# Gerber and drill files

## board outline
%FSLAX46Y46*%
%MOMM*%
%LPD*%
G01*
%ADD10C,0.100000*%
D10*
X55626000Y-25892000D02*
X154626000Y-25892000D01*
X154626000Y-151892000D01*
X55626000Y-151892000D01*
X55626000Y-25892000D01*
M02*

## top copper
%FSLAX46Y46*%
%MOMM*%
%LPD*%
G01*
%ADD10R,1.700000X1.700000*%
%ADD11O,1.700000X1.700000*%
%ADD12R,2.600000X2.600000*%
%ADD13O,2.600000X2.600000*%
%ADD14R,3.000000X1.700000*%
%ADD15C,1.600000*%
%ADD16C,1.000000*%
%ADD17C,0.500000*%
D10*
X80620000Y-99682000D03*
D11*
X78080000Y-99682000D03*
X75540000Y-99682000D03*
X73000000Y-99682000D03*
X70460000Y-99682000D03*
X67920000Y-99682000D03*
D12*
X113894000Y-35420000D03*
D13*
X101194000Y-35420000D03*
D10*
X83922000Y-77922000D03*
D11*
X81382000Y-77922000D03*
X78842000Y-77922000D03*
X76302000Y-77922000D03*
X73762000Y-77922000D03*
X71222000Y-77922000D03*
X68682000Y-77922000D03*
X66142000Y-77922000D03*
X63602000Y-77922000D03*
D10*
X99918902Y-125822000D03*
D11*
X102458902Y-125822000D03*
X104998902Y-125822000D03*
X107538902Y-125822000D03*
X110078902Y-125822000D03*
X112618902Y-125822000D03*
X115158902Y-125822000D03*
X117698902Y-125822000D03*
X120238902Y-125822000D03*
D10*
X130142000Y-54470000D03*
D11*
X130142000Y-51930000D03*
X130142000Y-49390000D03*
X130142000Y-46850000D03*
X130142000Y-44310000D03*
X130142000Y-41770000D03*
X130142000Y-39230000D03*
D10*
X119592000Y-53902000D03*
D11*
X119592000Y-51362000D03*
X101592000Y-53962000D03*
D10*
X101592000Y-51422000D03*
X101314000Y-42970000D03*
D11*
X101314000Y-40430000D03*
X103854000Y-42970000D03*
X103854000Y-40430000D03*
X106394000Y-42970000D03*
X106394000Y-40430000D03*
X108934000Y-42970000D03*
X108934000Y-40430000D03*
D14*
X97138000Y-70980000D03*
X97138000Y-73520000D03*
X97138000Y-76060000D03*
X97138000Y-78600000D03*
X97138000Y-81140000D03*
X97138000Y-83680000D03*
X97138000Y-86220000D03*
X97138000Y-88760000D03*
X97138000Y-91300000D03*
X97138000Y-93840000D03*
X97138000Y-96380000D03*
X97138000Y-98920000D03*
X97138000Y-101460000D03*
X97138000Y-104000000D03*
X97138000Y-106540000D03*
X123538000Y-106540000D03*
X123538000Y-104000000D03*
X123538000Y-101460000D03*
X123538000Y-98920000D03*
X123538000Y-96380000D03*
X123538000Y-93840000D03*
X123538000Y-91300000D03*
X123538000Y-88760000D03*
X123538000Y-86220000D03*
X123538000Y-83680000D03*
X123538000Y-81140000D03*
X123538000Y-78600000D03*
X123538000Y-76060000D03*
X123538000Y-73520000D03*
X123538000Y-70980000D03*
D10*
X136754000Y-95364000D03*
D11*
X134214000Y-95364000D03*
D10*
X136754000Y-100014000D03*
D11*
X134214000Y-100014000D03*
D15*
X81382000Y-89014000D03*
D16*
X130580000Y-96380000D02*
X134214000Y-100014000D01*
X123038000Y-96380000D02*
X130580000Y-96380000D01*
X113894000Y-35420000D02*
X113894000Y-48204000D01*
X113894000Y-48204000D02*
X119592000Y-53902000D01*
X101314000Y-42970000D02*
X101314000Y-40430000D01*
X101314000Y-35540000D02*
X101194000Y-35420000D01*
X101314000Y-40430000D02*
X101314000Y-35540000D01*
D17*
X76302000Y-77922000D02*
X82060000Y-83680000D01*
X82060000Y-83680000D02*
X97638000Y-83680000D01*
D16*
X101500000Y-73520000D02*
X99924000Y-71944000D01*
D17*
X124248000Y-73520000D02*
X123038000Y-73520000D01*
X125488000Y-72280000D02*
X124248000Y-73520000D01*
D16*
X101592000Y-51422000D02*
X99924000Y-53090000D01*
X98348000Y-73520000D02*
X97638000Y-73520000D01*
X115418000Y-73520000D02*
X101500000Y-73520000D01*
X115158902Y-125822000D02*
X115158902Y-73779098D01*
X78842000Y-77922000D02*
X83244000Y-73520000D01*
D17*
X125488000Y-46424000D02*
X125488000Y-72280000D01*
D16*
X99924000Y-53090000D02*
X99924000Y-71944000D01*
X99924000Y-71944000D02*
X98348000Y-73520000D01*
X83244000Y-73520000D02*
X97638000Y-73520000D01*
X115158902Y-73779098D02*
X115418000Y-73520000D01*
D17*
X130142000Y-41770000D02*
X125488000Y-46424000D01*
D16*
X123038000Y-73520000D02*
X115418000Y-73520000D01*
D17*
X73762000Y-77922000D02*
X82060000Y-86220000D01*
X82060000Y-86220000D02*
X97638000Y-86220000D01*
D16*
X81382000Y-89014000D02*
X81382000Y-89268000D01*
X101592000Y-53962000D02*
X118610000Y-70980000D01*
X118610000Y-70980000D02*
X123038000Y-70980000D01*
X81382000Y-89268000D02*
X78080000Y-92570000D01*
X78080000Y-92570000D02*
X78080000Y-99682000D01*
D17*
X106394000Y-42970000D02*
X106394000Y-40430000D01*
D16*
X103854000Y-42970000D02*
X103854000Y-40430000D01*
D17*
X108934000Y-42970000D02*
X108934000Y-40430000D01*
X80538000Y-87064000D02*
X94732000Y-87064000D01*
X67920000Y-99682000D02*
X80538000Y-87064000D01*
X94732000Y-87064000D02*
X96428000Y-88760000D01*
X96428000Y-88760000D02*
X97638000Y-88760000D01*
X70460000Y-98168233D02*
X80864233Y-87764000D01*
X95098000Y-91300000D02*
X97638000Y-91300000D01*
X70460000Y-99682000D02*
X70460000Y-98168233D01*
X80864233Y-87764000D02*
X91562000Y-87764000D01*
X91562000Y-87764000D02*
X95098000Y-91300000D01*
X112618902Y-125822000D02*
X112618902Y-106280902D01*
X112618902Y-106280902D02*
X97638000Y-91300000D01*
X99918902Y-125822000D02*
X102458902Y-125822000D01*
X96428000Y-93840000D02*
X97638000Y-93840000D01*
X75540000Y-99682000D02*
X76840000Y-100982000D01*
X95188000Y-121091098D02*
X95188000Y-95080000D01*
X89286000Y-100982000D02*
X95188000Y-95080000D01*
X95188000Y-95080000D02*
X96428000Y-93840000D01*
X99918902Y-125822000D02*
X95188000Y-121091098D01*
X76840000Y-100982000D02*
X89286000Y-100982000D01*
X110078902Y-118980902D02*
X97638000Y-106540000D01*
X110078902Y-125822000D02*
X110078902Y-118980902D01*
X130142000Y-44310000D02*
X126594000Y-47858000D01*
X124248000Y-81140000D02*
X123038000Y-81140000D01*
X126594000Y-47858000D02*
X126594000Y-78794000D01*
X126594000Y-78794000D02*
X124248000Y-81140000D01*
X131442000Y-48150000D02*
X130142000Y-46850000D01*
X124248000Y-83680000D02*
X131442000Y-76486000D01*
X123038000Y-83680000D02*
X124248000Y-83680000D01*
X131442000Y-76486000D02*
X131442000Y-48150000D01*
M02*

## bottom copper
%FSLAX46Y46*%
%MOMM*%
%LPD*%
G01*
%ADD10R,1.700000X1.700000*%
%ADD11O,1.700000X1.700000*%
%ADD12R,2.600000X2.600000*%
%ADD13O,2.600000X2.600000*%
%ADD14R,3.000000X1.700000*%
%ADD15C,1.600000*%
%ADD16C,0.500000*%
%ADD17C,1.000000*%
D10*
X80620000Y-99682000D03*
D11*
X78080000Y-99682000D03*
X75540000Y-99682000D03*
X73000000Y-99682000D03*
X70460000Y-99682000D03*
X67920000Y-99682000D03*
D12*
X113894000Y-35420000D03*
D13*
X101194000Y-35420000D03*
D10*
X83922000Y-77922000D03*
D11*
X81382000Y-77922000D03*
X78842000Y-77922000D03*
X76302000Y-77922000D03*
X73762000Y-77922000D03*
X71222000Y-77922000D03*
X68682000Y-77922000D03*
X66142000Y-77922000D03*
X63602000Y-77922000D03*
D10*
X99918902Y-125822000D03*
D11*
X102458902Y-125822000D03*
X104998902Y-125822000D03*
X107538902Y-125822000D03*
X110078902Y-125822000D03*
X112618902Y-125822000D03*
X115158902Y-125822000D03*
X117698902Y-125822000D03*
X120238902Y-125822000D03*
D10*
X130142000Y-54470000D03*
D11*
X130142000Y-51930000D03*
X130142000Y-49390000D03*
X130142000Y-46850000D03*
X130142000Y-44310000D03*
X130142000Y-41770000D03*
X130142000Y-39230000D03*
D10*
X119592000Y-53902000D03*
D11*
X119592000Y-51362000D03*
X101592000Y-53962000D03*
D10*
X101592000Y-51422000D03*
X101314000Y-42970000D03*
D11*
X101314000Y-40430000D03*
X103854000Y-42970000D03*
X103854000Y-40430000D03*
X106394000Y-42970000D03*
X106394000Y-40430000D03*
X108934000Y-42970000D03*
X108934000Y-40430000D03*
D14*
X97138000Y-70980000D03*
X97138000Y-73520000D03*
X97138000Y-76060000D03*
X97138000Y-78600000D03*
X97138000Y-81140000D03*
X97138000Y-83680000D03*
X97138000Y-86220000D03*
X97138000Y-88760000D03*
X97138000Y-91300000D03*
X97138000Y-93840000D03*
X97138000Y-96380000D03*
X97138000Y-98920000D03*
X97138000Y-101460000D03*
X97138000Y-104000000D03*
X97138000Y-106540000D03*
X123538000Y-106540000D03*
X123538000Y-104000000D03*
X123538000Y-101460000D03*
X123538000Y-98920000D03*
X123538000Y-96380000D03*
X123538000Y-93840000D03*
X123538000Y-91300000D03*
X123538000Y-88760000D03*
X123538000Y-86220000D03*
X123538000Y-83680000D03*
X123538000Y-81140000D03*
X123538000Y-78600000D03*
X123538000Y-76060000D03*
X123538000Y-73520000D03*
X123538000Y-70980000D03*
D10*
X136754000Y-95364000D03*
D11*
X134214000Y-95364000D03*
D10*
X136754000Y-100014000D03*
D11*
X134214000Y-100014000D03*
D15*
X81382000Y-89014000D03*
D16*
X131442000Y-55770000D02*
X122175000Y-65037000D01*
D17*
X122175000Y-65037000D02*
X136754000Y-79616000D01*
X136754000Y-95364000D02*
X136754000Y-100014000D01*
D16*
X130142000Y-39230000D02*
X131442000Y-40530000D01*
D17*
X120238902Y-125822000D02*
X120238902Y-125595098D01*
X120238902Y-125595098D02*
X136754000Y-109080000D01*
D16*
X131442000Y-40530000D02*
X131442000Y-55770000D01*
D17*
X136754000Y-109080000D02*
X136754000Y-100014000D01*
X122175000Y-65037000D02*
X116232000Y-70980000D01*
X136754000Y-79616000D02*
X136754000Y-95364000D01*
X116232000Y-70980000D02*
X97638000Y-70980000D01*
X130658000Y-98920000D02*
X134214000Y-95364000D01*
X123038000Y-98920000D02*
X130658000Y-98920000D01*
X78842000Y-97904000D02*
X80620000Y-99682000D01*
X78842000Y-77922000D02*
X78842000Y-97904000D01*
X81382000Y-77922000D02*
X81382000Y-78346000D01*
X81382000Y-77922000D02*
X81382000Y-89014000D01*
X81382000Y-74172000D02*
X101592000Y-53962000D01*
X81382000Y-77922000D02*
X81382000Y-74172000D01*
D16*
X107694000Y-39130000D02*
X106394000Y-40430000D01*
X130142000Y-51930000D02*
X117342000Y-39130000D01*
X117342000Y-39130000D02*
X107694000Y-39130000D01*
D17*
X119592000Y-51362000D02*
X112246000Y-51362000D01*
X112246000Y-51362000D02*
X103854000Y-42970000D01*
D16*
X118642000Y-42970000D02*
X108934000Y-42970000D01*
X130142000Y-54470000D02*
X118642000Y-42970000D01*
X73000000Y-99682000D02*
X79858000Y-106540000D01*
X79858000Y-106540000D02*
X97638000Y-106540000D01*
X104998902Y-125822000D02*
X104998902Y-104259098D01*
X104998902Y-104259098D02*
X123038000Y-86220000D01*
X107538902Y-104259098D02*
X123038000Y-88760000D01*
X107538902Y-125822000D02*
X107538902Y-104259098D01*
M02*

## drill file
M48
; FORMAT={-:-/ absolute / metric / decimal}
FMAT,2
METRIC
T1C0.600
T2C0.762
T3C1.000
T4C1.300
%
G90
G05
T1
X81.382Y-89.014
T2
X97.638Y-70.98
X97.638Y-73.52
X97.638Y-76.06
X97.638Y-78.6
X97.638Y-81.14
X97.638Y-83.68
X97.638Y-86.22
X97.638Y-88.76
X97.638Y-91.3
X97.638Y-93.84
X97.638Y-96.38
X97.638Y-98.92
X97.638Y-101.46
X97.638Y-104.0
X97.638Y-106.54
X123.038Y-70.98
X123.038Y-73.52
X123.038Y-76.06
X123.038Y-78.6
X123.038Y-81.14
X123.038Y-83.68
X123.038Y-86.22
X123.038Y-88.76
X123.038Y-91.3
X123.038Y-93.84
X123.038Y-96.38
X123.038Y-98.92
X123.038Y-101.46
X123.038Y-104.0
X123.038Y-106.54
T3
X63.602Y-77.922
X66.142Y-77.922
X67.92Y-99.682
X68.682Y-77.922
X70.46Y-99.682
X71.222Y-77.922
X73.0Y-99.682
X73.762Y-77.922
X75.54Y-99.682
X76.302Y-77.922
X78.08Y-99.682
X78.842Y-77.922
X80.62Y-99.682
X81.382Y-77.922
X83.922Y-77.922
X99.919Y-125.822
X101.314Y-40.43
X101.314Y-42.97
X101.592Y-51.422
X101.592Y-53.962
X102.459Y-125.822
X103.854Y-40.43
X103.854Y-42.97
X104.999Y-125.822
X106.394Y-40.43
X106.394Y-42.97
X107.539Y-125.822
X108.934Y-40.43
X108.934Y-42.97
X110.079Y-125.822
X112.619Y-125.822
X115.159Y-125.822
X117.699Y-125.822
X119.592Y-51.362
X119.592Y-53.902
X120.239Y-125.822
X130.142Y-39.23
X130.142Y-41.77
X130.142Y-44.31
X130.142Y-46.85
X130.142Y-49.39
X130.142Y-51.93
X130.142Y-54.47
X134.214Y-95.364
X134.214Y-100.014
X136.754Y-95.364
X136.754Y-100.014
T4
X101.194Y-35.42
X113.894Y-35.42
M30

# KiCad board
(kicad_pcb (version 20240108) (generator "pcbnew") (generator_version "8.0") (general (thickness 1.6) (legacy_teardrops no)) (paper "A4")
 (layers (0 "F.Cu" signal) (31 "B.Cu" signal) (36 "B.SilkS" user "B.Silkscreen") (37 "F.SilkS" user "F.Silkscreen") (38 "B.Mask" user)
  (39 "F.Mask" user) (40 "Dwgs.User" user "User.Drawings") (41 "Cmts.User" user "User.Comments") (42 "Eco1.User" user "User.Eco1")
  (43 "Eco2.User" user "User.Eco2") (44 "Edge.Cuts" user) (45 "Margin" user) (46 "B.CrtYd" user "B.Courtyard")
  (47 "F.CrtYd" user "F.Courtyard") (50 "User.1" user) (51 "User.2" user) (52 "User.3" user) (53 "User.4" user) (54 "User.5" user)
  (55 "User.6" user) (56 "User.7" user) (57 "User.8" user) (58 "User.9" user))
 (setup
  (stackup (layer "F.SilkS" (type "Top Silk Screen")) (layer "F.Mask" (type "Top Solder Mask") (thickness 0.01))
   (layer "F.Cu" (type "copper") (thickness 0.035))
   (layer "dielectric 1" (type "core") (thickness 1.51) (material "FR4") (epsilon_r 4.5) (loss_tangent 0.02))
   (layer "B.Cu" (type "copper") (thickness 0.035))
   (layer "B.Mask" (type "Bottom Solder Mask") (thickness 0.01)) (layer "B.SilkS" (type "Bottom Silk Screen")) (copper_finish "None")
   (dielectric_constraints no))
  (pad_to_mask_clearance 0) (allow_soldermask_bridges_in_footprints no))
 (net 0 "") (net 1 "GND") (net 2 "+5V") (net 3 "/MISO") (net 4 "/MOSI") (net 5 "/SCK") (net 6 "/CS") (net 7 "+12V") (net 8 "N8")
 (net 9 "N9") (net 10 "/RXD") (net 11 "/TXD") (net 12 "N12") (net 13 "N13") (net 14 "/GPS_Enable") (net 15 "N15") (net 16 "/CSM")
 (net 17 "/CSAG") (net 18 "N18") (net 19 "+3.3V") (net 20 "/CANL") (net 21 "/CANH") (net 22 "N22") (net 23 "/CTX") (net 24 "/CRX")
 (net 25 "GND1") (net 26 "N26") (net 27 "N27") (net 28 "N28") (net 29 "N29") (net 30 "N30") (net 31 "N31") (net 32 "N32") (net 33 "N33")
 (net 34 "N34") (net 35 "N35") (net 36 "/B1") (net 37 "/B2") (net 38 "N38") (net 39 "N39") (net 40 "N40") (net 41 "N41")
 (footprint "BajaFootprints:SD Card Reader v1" (layer "F.Cu") (at 74.27 117.462 90)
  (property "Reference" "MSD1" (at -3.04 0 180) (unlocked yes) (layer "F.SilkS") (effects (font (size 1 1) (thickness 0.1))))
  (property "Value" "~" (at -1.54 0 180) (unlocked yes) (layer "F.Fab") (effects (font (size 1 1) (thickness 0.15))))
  (pad "1" thru_hole rect (at 17.78 6.35 270) (size 1.7 1.7) (drill 1) (layers "*.Cu" "*.Mask") (remove_unused_layers no) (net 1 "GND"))
  (pad "2" thru_hole oval (at 17.78 3.81 270) (size 1.7 1.7) (drill 1) (layers "*.Cu" "*.Mask") (remove_unused_layers no) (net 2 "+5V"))
  (pad "3" thru_hole oval (at 17.78 1.27 270) (size 1.7 1.7) (drill 1) (layers "*.Cu" "*.Mask") (remove_unused_layers no) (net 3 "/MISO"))
  (pad "4" thru_hole oval (at 17.78 -1.27 270) (size 1.7 1.7) (drill 1) (layers "*.Cu" "*.Mask") (remove_unused_layers no) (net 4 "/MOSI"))
  (pad "5" thru_hole oval (at 17.78 -3.81 270) (size 1.7 1.7) (drill 1) (layers "*.Cu" "*.Mask") (remove_unused_layers no) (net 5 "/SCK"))
  (pad "6" thru_hole oval (at 17.78 -6.35 270) (size 1.7 1.7) (drill 1) (layers "*.Cu" "*.Mask") (remove_unused_layers no) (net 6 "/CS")))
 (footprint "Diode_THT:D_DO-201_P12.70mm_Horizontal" (layer "F.Cu") (at 113.894 35.42 180)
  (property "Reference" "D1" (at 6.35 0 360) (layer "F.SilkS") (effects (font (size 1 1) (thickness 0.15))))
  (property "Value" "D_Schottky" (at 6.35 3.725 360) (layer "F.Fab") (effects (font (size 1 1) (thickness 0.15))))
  (pad "1" thru_hole rect (at 0 0 180) (size 2.6 2.6) (drill 1.3) (layers "*.Cu" "*.Mask") (remove_unused_layers no) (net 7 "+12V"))
  (pad "2" thru_hole oval (at 12.7 0 180) (size 2.6 2.6) (drill 1.3) (layers "*.Cu" "*.Mask") (remove_unused_layers no) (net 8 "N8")))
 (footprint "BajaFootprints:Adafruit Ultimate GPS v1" (layer "F.Cu") (at 73.762 62.852 -90)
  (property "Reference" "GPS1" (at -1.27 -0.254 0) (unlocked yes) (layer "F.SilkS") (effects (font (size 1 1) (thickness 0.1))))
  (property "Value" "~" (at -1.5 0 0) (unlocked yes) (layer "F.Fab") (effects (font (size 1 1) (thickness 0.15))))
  (pad "1" thru_hole rect (at 15.07 -10.16 270) (size 1.7 1.7) (drill 1) (layers "*.Cu" "*.Mask") (remove_unused_layers no) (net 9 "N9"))
  (pad "2" thru_hole oval (at 15.07 -7.62 270) (size 1.7 1.7) (drill 1) (layers "*.Cu" "*.Mask") (remove_unused_layers no) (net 2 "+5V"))
  (pad "3" thru_hole oval (at 15.07 -5.08 270) (size 1.7 1.7) (drill 1) (layers "*.Cu" "*.Mask") (remove_unused_layers no) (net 1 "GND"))
  (pad "4" thru_hole oval (at 15.07 -2.54 270) (size 1.7 1.7) (drill 1) (layers "*.Cu" "*.Mask") (remove_unused_layers no) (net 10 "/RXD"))
  (pad "5" thru_hole oval (at 15.07 0 270) (size 1.7 1.7) (drill 1) (layers "*.Cu" "*.Mask") (remove_unused_layers no) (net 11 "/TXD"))
  (pad "6" thru_hole oval (at 15.07 2.54 270) (size 1.7 1.7) (drill 1) (layers "*.Cu" "*.Mask") (remove_unused_layers no) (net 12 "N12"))
  (pad "7" thru_hole oval (at 15.07 5.08 270) (size 1.7 1.7) (drill 1) (layers "*.Cu" "*.Mask") (remove_unused_layers no) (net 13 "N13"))
  (pad "8" thru_hole oval (at 15.07 7.62 270) (size 1.7 1.7) (drill 1) (layers "*.Cu" "*.Mask") (remove_unused_layers no)
   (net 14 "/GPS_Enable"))
  (pad "9" thru_hole oval (at 15.07 10.16 270) (size 1.7 1.7) (drill 1) (layers "*.Cu" "*.Mask") (remove_unused_layers no) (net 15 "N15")))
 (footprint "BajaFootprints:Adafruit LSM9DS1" (layer "F.Cu") (at 110.084 133.972 90)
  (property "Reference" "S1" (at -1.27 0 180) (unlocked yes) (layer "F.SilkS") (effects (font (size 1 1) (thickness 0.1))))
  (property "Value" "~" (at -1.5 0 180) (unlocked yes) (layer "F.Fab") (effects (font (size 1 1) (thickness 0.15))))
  (pad "1" thru_hole rect (at 8.15 -10.165098 90) (size 1.7 1.7) (drill 1) (layers "*.Cu" "*.Mask") (remove_unused_layers no)
   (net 3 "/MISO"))
  (pad "2" thru_hole oval (at 8.15 -7.625098 90) (size 1.7 1.7) (drill 1) (layers "*.Cu" "*.Mask") (remove_unused_layers no) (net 3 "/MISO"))
  (pad "3" thru_hole oval (at 8.15 -5.085098 90) (size 1.7 1.7) (drill 1) (layers "*.Cu" "*.Mask") (remove_unused_layers no) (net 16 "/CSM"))
  (pad "4" thru_hole oval (at 8.15 -2.545098 90) (size 1.7 1.7) (drill 1) (layers "*.Cu" "*.Mask") (remove_unused_layers no)
   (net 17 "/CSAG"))
  (pad "5" thru_hole oval (at 8.15 -0.005098 90) (size 1.7 1.7) (drill 1) (layers "*.Cu" "*.Mask") (remove_unused_layers no) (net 4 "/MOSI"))
  (pad "6" thru_hole oval (at 8.15 2.534902 90) (size 1.7 1.7) (drill 1) (layers "*.Cu" "*.Mask") (remove_unused_layers no) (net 5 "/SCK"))
  (pad "7" thru_hole oval (at 8.15 5.074902 90) (size 1.7 1.7) (drill 1) (layers "*.Cu" "*.Mask") (remove_unused_layers no) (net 1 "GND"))
  (pad "8" thru_hole oval (at 8.15 7.614902 90) (size 1.7 1.7) (drill 1) (layers "*.Cu" "*.Mask") (remove_unused_layers no) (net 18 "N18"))
  (pad "9" thru_hole oval (at 8.15 10.154902 90) (size 1.7 1.7) (drill 1) (layers "*.Cu" "*.Mask") (remove_unused_layers no)
   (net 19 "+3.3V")))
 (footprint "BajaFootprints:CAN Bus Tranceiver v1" (layer "F.Cu") (at 138.532 46.85 180)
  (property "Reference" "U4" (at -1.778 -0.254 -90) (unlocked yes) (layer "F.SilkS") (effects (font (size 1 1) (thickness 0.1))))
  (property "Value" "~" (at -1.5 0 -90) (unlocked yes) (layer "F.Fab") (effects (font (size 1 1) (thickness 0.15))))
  (pad "1" thru_hole rect (at 8.39 -7.62 180) (size 1.7 1.7) (drill 1) (layers "*.Cu" "*.Mask") (remove_unused_layers no) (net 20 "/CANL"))
  (pad "2" thru_hole oval (at 8.39 -5.08 180) (size 1.7 1.7) (drill 1) (layers "*.Cu" "*.Mask") (remove_unused_layers no) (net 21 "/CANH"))
  (pad "3" thru_hole oval (at 8.39 -2.54 180) (size 1.7 1.7) (drill 1) (layers "*.Cu" "*.Mask") (remove_unused_layers no) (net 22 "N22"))
  (pad "4" thru_hole oval (at 8.39 0 180) (size 1.7 1.7) (drill 1) (layers "*.Cu" "*.Mask") (remove_unused_layers no) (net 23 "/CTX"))
  (pad "5" thru_hole oval (at 8.39 2.54 180) (size 1.7 1.7) (drill 1) (layers "*.Cu" "*.Mask") (remove_unused_layers no) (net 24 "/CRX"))
  (pad "6" thru_hole oval (at 8.39 5.08 180) (size 1.7 1.7) (drill 1) (layers "*.Cu" "*.Mask") (remove_unused_layers no) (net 1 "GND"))
  (pad "7" thru_hole oval (at 8.39 7.62 180) (size 1.7 1.7) (drill 1) (layers "*.Cu" "*.Mask") (remove_unused_layers no) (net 19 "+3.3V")))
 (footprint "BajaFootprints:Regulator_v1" (layer "F.Cu") (at 110.592 52.692 180)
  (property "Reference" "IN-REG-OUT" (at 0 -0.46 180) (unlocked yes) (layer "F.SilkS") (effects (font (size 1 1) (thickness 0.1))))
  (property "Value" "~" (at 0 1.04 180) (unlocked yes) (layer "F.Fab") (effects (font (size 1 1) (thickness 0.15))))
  (pad "1" thru_hole rect (at -9 -1.21 180) (size 1.7 1.7) (drill 1) (layers "*.Cu" "*.Mask") (remove_unused_layers no) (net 7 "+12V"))
  (pad "2" thru_hole oval (at -9 1.33 180) (size 1.7 1.7) (drill 1) (layers "*.Cu" "*.Mask") (remove_unused_layers no) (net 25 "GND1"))
  (pad "3" thru_hole oval (at 9 -1.27) (size 1.7 1.7) (drill 1) (layers "*.Cu" "*.Mask") (remove_unused_layers no) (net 2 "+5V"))
  (pad "4" thru_hole rect (at 9 1.27) (size 1.7 1.7) (drill 1) (layers "*.Cu" "*.Mask") (remove_unused_layers no) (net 1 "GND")))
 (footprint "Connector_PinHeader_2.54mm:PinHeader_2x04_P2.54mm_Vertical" (layer "F.Cu") (at 101.314 42.97 90)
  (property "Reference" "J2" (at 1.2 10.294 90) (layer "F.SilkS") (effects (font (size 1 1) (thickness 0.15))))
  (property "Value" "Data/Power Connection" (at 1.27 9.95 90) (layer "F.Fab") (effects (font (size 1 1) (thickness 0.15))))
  (pad "1" thru_hole rect (at 0 0 90) (size 1.7 1.7) (drill 1) (layers "*.Cu" "*.Mask") (remove_unused_layers no) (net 8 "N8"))
  (pad "2" thru_hole oval (at 2.54 0 90) (size 1.7 1.7) (drill 1) (layers "*.Cu" "*.Mask") (remove_unused_layers no) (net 8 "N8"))
  (pad "3" thru_hole oval (at 0 2.54 90) (size 1.7 1.7) (drill 1) (layers "*.Cu" "*.Mask") (remove_unused_layers no) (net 25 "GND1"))
  (pad "4" thru_hole oval (at 2.54 2.54 90) (size 1.7 1.7) (drill 1) (layers "*.Cu" "*.Mask") (remove_unused_layers no) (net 25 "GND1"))
  (pad "5" thru_hole oval (at 0 5.08 90) (size 1.7 1.7) (drill 1) (layers "*.Cu" "*.Mask") (remove_unused_layers no) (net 21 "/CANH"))
  (pad "6" thru_hole oval (at 2.54 5.08 90) (size 1.7 1.7) (drill 1) (layers "*.Cu" "*.Mask") (remove_unused_layers no) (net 21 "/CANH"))
  (pad "7" thru_hole oval (at 0 7.62 90) (size 1.7 1.7) (drill 1) (layers "*.Cu" "*.Mask") (remove_unused_layers no) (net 20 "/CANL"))
  (pad "8" thru_hole oval (at 2.54 7.62 90) (size 1.7 1.7) (drill 1) (layers "*.Cu" "*.Mask") (remove_unused_layers no) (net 20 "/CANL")))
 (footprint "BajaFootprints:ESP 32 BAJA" (layer "F.Cu") (at 110.338 70.98)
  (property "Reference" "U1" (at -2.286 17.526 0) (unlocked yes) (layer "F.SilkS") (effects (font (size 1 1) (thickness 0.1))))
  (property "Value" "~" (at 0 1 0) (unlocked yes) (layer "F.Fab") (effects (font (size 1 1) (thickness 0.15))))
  (pad "1" thru_hole rect (at -12.7 0) (size 3 1.7) (drill 0.762 (offset -0.5 0)) (layers "*.Cu" "*.Mask") (remove_unused_layers no)
   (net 19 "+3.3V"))
  (pad "2" thru_hole rect (at -12.7 2.54) (size 3 1.7) (drill 0.762 (offset -0.5 0)) (layers "*.Cu" "*.Mask") (remove_unused_layers no)
   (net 1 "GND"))
  (pad "3" thru_hole rect (at -12.7 5.08) (size 3 1.7) (drill 0.762 (offset -0.5 0)) (layers "*.Cu" "*.Mask") (remove_unused_layers no)
   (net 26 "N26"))
  (pad "4" thru_hole rect (at -12.7 7.62) (size 3 1.7) (drill 0.762 (offset -0.5 0)) (layers "*.Cu" "*.Mask") (remove_unused_layers no)
   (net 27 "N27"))
  (pad "5" thru_hole rect (at -12.7 10.16) (size 3 1.7) (drill 0.762 (offset -0.5 0)) (layers "*.Cu" "*.Mask") (remove_unused_layers no)
   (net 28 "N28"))
  (pad "6" thru_hole rect (at -12.7 12.7) (size 3 1.7) (drill 0.762 (offset -0.5 0)) (layers "*.Cu" "*.Mask") (remove_unused_layers no)
   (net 10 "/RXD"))
  (pad "7" thru_hole rect (at -12.7 15.24) (size 3 1.7) (drill 0.762 (offset -0.5 0)) (layers "*.Cu" "*.Mask") (remove_unused_layers no)
   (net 11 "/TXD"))
  (pad "8" thru_hole rect (at -12.7 17.78) (size 3 1.7) (drill 0.762 (offset -0.5 0)) (layers "*.Cu" "*.Mask") (remove_unused_layers no)
   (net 6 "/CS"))
  (pad "9" thru_hole rect (at -12.7 20.32) (size 3 1.7) (drill 0.762 (offset -0.5 0)) (layers "*.Cu" "*.Mask") (remove_unused_layers no)
   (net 5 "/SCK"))
  (pad "10" thru_hole rect (at -12.7 22.86) (size 3 1.7) (drill 0.762 (offset -0.5 0)) (layers "*.Cu" "*.Mask") (remove_unused_layers no)
   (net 3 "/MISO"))
  (pad "11" thru_hole rect (at -12.7 25.4) (size 3 1.7) (drill 0.762 (offset -0.5 0)) (layers "*.Cu" "*.Mask") (remove_unused_layers no)
   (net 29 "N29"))
  (pad "12" thru_hole rect (at -12.7 27.94) (size 3 1.7) (drill 0.762 (offset -0.5 0)) (layers "*.Cu" "*.Mask") (remove_unused_layers no)
   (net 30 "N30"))
  (pad "13" thru_hole rect (at -12.7 30.48) (size 3 1.7) (drill 0.762 (offset -0.5 0)) (layers "*.Cu" "*.Mask") (remove_unused_layers no)
   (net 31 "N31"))
  (pad "14" thru_hole rect (at -12.7 33.02) (size 3 1.7) (drill 0.762 (offset -0.5 0)) (layers "*.Cu" "*.Mask") (remove_unused_layers no)
   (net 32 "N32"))
  (pad "15" thru_hole rect (at -12.7 35.56) (size 3 1.7) (drill 0.762 (offset -0.5 0)) (layers "*.Cu" "*.Mask") (remove_unused_layers no)
   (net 4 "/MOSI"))
  (pad "16" thru_hole rect (at 12.7 35.56) (size 3 1.7) (drill 0.762 (offset 0.5 0)) (layers "*.Cu" "*.Mask") (remove_unused_layers no)
   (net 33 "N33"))
  (pad "17" thru_hole rect (at 12.7 33.02) (size 3 1.7) (drill 0.762 (offset 0.5 0)) (layers "*.Cu" "*.Mask") (remove_unused_layers no)
   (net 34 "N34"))
  (pad "18" thru_hole rect (at 12.7 30.48) (size 3 1.7) (drill 0.762 (offset 0.5 0)) (layers "*.Cu" "*.Mask") (remove_unused_layers no)
   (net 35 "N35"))
  (pad "19" thru_hole rect (at 12.7 27.94) (size 3 1.7) (drill 0.762 (offset 0.5 0)) (layers "*.Cu" "*.Mask") (remove_unused_layers no)
   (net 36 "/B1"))
  (pad "20" thru_hole rect (at 12.7 25.4) (size 3 1.7) (drill 0.762 (offset 0.5 0)) (layers "*.Cu" "*.Mask") (remove_unused_layers no)
   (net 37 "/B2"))
  (pad "21" thru_hole rect (at 12.7 22.86) (size 3 1.7) (drill 0.762 (offset 0.5 0)) (layers "*.Cu" "*.Mask") (remove_unused_layers no)
   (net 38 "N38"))
  (pad "22" thru_hole rect (at 12.7 20.32) (size 3 1.7) (drill 0.762 (offset 0.5 0)) (layers "*.Cu" "*.Mask") (remove_unused_layers no)
   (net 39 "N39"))
  (pad "23" thru_hole rect (at 12.7 17.78) (size 3 1.7) (drill 0.762 (offset 0.5 0)) (layers "*.Cu" "*.Mask") (remove_unused_layers no)
   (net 17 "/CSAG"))
  (pad "24" thru_hole rect (at 12.7 15.24) (size 3 1.7) (drill 0.762 (offset 0.5 0)) (layers "*.Cu" "*.Mask") (remove_unused_layers no)
   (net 16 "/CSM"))
  (pad "25" thru_hole rect (at 12.7 12.7) (size 3 1.7) (drill 0.762 (offset 0.5 0)) (layers "*.Cu" "*.Mask") (remove_unused_layers no)
   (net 23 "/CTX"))
  (pad "26" thru_hole rect (at 12.7 10.16) (size 3 1.7) (drill 0.762 (offset 0.5 0)) (layers "*.Cu" "*.Mask") (remove_unused_layers no)
   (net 24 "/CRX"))
  (pad "27" thru_hole rect (at 12.7 7.62) (size 3 1.7) (drill 0.762 (offset 0.5 0)) (layers "*.Cu" "*.Mask") (remove_unused_layers no)
   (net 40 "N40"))
  (pad "28" thru_hole rect (at 12.7 5.08) (size 3 1.7) (drill 0.762 (offset 0.5 0)) (layers "*.Cu" "*.Mask") (remove_unused_layers no)
   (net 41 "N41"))
  (pad "29" thru_hole rect (at 12.7 2.54) (size 3 1.7) (drill 0.762 (offset 0.5 0)) (layers "*.Cu" "*.Mask") (remove_unused_layers no)
   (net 1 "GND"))
  (pad "30" thru_hole rect (at 12.7 0) (size 3 1.7) (drill 0.762 (offset 0.5 0)) (layers "*.Cu" "*.Mask") (remove_unused_layers no)
   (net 2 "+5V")))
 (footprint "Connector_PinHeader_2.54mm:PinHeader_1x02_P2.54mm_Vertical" (layer "F.Cu") (at 136.754 95.364 -90)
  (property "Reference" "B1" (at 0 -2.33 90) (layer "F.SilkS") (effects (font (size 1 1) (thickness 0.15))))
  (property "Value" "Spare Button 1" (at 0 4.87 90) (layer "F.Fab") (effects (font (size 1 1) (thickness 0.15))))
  (pad "1" thru_hole rect (at 0 0 270) (size 1.7 1.7) (drill 1) (layers "*.Cu" "*.Mask") (remove_unused_layers no) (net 19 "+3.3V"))
  (pad "2" thru_hole oval (at 0 2.54 270) (size 1.7 1.7) (drill 1) (layers "*.Cu" "*.Mask") (remove_unused_layers no) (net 36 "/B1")))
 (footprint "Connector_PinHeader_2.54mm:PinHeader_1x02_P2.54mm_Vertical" (layer "F.Cu") (at 136.754 100.014 -90)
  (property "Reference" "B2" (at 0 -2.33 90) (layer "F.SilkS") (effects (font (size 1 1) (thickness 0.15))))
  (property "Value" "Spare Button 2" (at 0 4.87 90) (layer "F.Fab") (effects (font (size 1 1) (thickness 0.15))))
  (pad "1" thru_hole rect (at 0 0 270) (size 1.7 1.7) (drill 1) (layers "*.Cu" "*.Mask") (remove_unused_layers no) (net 19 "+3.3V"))
  (pad "2" thru_hole oval (at 0 2.54 270) (size 1.7 1.7) (drill 1) (layers "*.Cu" "*.Mask") (remove_unused_layers no) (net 37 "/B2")))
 (gr_rect (start 55.626 25.892) (end 154.626 151.892) (stroke (width 0.1) (type default)) (fill none) (layer "Edge.Cuts"))
 (segment (start 131.442 55.77) (end 122.175 65.037) (width 0.5) (layer "B.Cu") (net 19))
 (segment (start 122.175 65.037) (end 136.754 79.616) (width 1) (layer "B.Cu") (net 19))
 (segment (start 136.754 95.364) (end 136.754 100.014) (width 1) (layer "B.Cu") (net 19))
 (segment (start 130.142 39.23) (end 131.442 40.53) (width 0.5) (layer "B.Cu") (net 19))
 (segment (start 120.238902 125.822) (end 120.238902 125.595098) (width 1) (layer "B.Cu") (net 19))
 (segment (start 120.238902 125.595098) (end 136.754 109.08) (width 1) (layer "B.Cu") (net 19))
 (segment (start 131.442 40.53) (end 131.442 55.77) (width 0.5) (layer "B.Cu") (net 19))
 (segment (start 136.754 109.08) (end 136.754 100.014) (width 1) (layer "B.Cu") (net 19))
 (segment (start 122.175 65.037) (end 116.232 70.98) (width 1) (layer "B.Cu") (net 19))
 (segment (start 136.754 79.616) (end 136.754 95.364) (width 1) (layer "B.Cu") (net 19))
 (segment (start 116.232 70.98) (end 97.638 70.98) (width 1) (layer "B.Cu") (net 19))
 (segment (start 130.658 98.92) (end 134.214 95.364) (width 1) (layer "B.Cu") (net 36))
 (segment (start 123.038 98.92) (end 130.658 98.92) (width 1) (layer "B.Cu") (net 36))
 (segment (start 130.58 96.38) (end 134.214 100.014) (width 1) (layer "F.Cu") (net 37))
 (segment (start 123.038 96.38) (end 130.58 96.38) (width 1) (layer "F.Cu") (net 37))
 (segment (start 113.894 35.42) (end 113.894 48.204) (width 1) (layer "F.Cu") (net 7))
 (segment (start 113.894 48.204) (end 119.592 53.902) (width 1) (layer "F.Cu") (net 7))
 (segment (start 101.314 42.97) (end 101.314 40.43) (width 1) (layer "F.Cu") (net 8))
 (segment (start 101.314 35.54) (end 101.194 35.42) (width 1) (layer "F.Cu") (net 8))
 (segment (start 101.314 40.43) (end 101.314 35.54) (width 1) (layer "F.Cu") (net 8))
 (segment (start 76.302 77.922) (end 82.06 83.68) (width 0.5) (layer "F.Cu") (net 10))
 (segment (start 82.06 83.68) (end 97.638 83.68) (width 0.5) (layer "F.Cu") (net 10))
 (segment (start 101.5 73.52) (end 99.924 71.944) (width 1) (layer "F.Cu") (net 1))
 (segment (start 124.248 73.52) (end 123.038 73.52) (width 0.5) (layer "F.Cu") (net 1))
 (segment (start 125.488 72.28) (end 124.248 73.52) (width 0.5) (layer "F.Cu") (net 1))
 (segment (start 101.592 51.422) (end 99.924 53.09) (width 1) (layer "F.Cu") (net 1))
 (segment (start 98.348 73.52) (end 97.638 73.52) (width 1) (layer "F.Cu") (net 1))
 (segment (start 115.418 73.52) (end 101.5 73.52) (width 1) (layer "F.Cu") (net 1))
 (segment (start 115.158902 125.822) (end 115.158902 73.779098) (width 1) (layer "F.Cu") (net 1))
 (segment (start 78.842 77.922) (end 83.244 73.52) (width 1) (layer "F.Cu") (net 1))
 (segment (start 125.488 46.424) (end 125.488 72.28) (width 0.5) (layer "F.Cu") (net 1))
 (segment (start 99.924 53.09) (end 99.924 71.944) (width 1) (layer "F.Cu") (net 1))
 (segment (start 99.924 71.944) (end 98.348 73.52) (width 1) (layer "F.Cu") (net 1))
 (segment (start 83.244 73.52) (end 97.638 73.52) (width 1) (layer "F.Cu") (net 1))
 (segment (start 115.158902 73.779098) (end 115.418 73.52) (width 1) (layer "F.Cu") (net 1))
 (segment (start 130.142 41.77) (end 125.488 46.424) (width 0.5) (layer "F.Cu") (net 1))
 (segment (start 123.038 73.52) (end 115.418 73.52) (width 1) (layer "F.Cu") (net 1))
 (segment (start 78.842 97.904) (end 80.62 99.682) (width 1) (layer "B.Cu") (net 1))
 (segment (start 78.842 77.922) (end 78.842 97.904) (width 1) (layer "B.Cu") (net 1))
 (segment (start 73.762 77.922) (end 82.06 86.22) (width 0.5) (layer "F.Cu") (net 11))
 (segment (start 82.06 86.22) (end 97.638 86.22) (width 0.5) (layer "F.Cu") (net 11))
 (segment (start 81.382 89.014) (end 81.382 89.268) (width 1) (layer "F.Cu") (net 2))
 (segment (start 101.592 53.962) (end 118.61 70.98) (width 1) (layer "F.Cu") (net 2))
 (segment (start 118.61 70.98) (end 123.038 70.98) (width 1) (layer "F.Cu") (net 2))
 (segment (start 81.382 89.268) (end 78.08 92.57) (width 1) (layer "F.Cu") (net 2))
 (segment (start 78.08 92.57) (end 78.08 99.682) (width 1) (layer "F.Cu") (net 2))
 (via (at 81.382 89.014) (size 1.6) (drill 0.6) (layers "F.Cu" "B.Cu") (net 2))
 (segment (start 81.382 77.922) (end 81.382 78.346) (width 1) (layer "B.Cu") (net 2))
 (segment (start 81.382 77.922) (end 81.382 89.014) (width 1) (layer "B.Cu") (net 2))
 (segment (start 81.382 74.172) (end 101.592 53.962) (width 1) (layer "B.Cu") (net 2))
 (segment (start 81.382 77.922) (end 81.382 74.172) (width 1) (layer "B.Cu") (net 2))
 (segment (start 106.394 42.97) (end 106.394 40.43) (width 0.5) (layer "F.Cu") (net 21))
 (segment (start 107.694 39.13) (end 106.394 40.43) (width 0.5) (layer "B.Cu") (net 21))
 (segment (start 130.142 51.93) (end 117.342 39.13) (width 0.5) (layer "B.Cu") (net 21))
 (segment (start 117.342 39.13) (end 107.694 39.13) (width 0.5) (layer "B.Cu") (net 21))
 (segment (start 103.854 42.97) (end 103.854 40.43) (width 1) (layer "F.Cu") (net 25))
 (segment (start 119.592 51.362) (end 112.246 51.362) (width 1) (layer "B.Cu") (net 25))
 (segment (start 112.246 51.362) (end 103.854 42.97) (width 1) (layer "B.Cu") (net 25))
 (segment (start 108.934 42.97) (end 108.934 40.43) (width 0.5) (layer "F.Cu") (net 20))
 (segment (start 118.642 42.97) (end 108.934 42.97) (width 0.5) (layer "B.Cu") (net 20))
 (segment (start 130.142 54.47) (end 118.642 42.97) (width 0.5) (layer "B.Cu") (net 20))
 (segment (start 80.538 87.064) (end 94.732 87.064) (width 0.5) (layer "F.Cu") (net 6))
 (segment (start 67.92 99.682) (end 80.538 87.064) (width 0.5) (layer "F.Cu") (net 6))
 (segment (start 94.732 87.064) (end 96.428 88.76) (width 0.5) (layer "F.Cu") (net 6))
 (segment (start 96.428 88.76) (end 97.638 88.76) (width 0.5) (layer "F.Cu") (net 6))
 (segment (start 70.46 98.168233) (end 80.864233 87.764) (width 0.5) (layer "F.Cu") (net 5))
 (segment (start 95.098 91.3) (end 97.638 91.3) (width 0.5) (layer "F.Cu") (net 5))
 (segment (start 70.46 99.682) (end 70.46 98.168233) (width 0.5) (layer "F.Cu") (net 5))
 (segment (start 80.864233 87.764) (end 91.562 87.764) (width 0.5) (layer "F.Cu") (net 5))
 (segment (start 91.562 87.764) (end 95.098 91.3) (width 0.5) (layer "F.Cu") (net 5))
 (segment (start 112.618902 125.822) (end 112.618902 106.280902) (width 0.5) (layer "F.Cu") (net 5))
 (segment (start 112.618902 106.280902) (end 97.638 91.3) (width 0.5) (layer "F.Cu") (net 5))
 (segment (start 99.918902 125.822) (end 102.458902 125.822) (width 0.5) (layer "F.Cu") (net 3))
 (segment (start 96.428 93.84) (end 97.638 93.84) (width 0.5) (layer "F.Cu") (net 3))
 (segment (start 75.54 99.682) (end 76.84 100.982) (width 0.5) (layer "F.Cu") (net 3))
 (segment (start 95.188 121.091098) (end 95.188 95.08) (width 0.5) (layer "F.Cu") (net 3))
 (segment (start 89.286 100.982) (end 95.188 95.08) (width 0.5) (layer "F.Cu") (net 3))
 (segment (start 95.188 95.08) (end 96.428 93.84) (width 0.5) (layer "F.Cu") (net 3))
 (segment (start 99.918902 125.822) (end 95.188 121.091098) (width 0.5) (layer "F.Cu") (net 3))
 (segment (start 76.84 100.982) (end 89.286 100.982) (width 0.5) (layer "F.Cu") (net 3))
 (segment (start 110.078902 118.980902) (end 97.638 106.54) (width 0.5) (layer "F.Cu") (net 4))
 (segment (start 110.078902 125.822) (end 110.078902 118.980902) (width 0.5) (layer "F.Cu") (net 4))
 (segment (start 73 99.682) (end 79.858 106.54) (width 0.5) (layer "B.Cu") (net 4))
 (segment (start 79.858 106.54) (end 97.638 106.54) (width 0.5) (layer "B.Cu") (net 4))
 (segment (start 104.998902 125.822) (end 104.998902 104.259098) (width 0.5) (layer "B.Cu") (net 16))
 (segment (start 104.998902 104.259098) (end 123.038 86.22) (width 0.5) (layer "B.Cu") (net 16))
 (segment (start 107.538902 104.259098) (end 123.038 88.76) (width 0.5) (layer "B.Cu") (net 17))
 (segment (start 107.538902 125.822) (end 107.538902 104.259098) (width 0.5) (layer "B.Cu") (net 17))
 (segment (start 130.142 44.31) (end 126.594 47.858) (width 0.5) (layer "F.Cu") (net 24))
 (segment (start 124.248 81.14) (end 123.038 81.14) (width 0.5) (layer "F.Cu") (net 24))
 (segment (start 126.594 47.858) (end 126.594 78.794) (width 0.5) (layer "F.Cu") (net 24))
 (segment (start 126.594 78.794) (end 124.248 81.14) (width 0.5) (layer "F.Cu") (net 24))
 (segment (start 131.442 48.15) (end 130.142 46.85) (width 0.5) (layer "F.Cu") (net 23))
 (segment (start 124.248 83.68) (end 131.442 76.486) (width 0.5) (layer "F.Cu") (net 23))
 (segment (start 123.038 83.68) (end 124.248 83.68) (width 0.5) (layer "F.Cu") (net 23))
 (segment (start 131.442 76.486) (end 131.442 48.15) (width 0.5) (layer "F.Cu") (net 23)))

